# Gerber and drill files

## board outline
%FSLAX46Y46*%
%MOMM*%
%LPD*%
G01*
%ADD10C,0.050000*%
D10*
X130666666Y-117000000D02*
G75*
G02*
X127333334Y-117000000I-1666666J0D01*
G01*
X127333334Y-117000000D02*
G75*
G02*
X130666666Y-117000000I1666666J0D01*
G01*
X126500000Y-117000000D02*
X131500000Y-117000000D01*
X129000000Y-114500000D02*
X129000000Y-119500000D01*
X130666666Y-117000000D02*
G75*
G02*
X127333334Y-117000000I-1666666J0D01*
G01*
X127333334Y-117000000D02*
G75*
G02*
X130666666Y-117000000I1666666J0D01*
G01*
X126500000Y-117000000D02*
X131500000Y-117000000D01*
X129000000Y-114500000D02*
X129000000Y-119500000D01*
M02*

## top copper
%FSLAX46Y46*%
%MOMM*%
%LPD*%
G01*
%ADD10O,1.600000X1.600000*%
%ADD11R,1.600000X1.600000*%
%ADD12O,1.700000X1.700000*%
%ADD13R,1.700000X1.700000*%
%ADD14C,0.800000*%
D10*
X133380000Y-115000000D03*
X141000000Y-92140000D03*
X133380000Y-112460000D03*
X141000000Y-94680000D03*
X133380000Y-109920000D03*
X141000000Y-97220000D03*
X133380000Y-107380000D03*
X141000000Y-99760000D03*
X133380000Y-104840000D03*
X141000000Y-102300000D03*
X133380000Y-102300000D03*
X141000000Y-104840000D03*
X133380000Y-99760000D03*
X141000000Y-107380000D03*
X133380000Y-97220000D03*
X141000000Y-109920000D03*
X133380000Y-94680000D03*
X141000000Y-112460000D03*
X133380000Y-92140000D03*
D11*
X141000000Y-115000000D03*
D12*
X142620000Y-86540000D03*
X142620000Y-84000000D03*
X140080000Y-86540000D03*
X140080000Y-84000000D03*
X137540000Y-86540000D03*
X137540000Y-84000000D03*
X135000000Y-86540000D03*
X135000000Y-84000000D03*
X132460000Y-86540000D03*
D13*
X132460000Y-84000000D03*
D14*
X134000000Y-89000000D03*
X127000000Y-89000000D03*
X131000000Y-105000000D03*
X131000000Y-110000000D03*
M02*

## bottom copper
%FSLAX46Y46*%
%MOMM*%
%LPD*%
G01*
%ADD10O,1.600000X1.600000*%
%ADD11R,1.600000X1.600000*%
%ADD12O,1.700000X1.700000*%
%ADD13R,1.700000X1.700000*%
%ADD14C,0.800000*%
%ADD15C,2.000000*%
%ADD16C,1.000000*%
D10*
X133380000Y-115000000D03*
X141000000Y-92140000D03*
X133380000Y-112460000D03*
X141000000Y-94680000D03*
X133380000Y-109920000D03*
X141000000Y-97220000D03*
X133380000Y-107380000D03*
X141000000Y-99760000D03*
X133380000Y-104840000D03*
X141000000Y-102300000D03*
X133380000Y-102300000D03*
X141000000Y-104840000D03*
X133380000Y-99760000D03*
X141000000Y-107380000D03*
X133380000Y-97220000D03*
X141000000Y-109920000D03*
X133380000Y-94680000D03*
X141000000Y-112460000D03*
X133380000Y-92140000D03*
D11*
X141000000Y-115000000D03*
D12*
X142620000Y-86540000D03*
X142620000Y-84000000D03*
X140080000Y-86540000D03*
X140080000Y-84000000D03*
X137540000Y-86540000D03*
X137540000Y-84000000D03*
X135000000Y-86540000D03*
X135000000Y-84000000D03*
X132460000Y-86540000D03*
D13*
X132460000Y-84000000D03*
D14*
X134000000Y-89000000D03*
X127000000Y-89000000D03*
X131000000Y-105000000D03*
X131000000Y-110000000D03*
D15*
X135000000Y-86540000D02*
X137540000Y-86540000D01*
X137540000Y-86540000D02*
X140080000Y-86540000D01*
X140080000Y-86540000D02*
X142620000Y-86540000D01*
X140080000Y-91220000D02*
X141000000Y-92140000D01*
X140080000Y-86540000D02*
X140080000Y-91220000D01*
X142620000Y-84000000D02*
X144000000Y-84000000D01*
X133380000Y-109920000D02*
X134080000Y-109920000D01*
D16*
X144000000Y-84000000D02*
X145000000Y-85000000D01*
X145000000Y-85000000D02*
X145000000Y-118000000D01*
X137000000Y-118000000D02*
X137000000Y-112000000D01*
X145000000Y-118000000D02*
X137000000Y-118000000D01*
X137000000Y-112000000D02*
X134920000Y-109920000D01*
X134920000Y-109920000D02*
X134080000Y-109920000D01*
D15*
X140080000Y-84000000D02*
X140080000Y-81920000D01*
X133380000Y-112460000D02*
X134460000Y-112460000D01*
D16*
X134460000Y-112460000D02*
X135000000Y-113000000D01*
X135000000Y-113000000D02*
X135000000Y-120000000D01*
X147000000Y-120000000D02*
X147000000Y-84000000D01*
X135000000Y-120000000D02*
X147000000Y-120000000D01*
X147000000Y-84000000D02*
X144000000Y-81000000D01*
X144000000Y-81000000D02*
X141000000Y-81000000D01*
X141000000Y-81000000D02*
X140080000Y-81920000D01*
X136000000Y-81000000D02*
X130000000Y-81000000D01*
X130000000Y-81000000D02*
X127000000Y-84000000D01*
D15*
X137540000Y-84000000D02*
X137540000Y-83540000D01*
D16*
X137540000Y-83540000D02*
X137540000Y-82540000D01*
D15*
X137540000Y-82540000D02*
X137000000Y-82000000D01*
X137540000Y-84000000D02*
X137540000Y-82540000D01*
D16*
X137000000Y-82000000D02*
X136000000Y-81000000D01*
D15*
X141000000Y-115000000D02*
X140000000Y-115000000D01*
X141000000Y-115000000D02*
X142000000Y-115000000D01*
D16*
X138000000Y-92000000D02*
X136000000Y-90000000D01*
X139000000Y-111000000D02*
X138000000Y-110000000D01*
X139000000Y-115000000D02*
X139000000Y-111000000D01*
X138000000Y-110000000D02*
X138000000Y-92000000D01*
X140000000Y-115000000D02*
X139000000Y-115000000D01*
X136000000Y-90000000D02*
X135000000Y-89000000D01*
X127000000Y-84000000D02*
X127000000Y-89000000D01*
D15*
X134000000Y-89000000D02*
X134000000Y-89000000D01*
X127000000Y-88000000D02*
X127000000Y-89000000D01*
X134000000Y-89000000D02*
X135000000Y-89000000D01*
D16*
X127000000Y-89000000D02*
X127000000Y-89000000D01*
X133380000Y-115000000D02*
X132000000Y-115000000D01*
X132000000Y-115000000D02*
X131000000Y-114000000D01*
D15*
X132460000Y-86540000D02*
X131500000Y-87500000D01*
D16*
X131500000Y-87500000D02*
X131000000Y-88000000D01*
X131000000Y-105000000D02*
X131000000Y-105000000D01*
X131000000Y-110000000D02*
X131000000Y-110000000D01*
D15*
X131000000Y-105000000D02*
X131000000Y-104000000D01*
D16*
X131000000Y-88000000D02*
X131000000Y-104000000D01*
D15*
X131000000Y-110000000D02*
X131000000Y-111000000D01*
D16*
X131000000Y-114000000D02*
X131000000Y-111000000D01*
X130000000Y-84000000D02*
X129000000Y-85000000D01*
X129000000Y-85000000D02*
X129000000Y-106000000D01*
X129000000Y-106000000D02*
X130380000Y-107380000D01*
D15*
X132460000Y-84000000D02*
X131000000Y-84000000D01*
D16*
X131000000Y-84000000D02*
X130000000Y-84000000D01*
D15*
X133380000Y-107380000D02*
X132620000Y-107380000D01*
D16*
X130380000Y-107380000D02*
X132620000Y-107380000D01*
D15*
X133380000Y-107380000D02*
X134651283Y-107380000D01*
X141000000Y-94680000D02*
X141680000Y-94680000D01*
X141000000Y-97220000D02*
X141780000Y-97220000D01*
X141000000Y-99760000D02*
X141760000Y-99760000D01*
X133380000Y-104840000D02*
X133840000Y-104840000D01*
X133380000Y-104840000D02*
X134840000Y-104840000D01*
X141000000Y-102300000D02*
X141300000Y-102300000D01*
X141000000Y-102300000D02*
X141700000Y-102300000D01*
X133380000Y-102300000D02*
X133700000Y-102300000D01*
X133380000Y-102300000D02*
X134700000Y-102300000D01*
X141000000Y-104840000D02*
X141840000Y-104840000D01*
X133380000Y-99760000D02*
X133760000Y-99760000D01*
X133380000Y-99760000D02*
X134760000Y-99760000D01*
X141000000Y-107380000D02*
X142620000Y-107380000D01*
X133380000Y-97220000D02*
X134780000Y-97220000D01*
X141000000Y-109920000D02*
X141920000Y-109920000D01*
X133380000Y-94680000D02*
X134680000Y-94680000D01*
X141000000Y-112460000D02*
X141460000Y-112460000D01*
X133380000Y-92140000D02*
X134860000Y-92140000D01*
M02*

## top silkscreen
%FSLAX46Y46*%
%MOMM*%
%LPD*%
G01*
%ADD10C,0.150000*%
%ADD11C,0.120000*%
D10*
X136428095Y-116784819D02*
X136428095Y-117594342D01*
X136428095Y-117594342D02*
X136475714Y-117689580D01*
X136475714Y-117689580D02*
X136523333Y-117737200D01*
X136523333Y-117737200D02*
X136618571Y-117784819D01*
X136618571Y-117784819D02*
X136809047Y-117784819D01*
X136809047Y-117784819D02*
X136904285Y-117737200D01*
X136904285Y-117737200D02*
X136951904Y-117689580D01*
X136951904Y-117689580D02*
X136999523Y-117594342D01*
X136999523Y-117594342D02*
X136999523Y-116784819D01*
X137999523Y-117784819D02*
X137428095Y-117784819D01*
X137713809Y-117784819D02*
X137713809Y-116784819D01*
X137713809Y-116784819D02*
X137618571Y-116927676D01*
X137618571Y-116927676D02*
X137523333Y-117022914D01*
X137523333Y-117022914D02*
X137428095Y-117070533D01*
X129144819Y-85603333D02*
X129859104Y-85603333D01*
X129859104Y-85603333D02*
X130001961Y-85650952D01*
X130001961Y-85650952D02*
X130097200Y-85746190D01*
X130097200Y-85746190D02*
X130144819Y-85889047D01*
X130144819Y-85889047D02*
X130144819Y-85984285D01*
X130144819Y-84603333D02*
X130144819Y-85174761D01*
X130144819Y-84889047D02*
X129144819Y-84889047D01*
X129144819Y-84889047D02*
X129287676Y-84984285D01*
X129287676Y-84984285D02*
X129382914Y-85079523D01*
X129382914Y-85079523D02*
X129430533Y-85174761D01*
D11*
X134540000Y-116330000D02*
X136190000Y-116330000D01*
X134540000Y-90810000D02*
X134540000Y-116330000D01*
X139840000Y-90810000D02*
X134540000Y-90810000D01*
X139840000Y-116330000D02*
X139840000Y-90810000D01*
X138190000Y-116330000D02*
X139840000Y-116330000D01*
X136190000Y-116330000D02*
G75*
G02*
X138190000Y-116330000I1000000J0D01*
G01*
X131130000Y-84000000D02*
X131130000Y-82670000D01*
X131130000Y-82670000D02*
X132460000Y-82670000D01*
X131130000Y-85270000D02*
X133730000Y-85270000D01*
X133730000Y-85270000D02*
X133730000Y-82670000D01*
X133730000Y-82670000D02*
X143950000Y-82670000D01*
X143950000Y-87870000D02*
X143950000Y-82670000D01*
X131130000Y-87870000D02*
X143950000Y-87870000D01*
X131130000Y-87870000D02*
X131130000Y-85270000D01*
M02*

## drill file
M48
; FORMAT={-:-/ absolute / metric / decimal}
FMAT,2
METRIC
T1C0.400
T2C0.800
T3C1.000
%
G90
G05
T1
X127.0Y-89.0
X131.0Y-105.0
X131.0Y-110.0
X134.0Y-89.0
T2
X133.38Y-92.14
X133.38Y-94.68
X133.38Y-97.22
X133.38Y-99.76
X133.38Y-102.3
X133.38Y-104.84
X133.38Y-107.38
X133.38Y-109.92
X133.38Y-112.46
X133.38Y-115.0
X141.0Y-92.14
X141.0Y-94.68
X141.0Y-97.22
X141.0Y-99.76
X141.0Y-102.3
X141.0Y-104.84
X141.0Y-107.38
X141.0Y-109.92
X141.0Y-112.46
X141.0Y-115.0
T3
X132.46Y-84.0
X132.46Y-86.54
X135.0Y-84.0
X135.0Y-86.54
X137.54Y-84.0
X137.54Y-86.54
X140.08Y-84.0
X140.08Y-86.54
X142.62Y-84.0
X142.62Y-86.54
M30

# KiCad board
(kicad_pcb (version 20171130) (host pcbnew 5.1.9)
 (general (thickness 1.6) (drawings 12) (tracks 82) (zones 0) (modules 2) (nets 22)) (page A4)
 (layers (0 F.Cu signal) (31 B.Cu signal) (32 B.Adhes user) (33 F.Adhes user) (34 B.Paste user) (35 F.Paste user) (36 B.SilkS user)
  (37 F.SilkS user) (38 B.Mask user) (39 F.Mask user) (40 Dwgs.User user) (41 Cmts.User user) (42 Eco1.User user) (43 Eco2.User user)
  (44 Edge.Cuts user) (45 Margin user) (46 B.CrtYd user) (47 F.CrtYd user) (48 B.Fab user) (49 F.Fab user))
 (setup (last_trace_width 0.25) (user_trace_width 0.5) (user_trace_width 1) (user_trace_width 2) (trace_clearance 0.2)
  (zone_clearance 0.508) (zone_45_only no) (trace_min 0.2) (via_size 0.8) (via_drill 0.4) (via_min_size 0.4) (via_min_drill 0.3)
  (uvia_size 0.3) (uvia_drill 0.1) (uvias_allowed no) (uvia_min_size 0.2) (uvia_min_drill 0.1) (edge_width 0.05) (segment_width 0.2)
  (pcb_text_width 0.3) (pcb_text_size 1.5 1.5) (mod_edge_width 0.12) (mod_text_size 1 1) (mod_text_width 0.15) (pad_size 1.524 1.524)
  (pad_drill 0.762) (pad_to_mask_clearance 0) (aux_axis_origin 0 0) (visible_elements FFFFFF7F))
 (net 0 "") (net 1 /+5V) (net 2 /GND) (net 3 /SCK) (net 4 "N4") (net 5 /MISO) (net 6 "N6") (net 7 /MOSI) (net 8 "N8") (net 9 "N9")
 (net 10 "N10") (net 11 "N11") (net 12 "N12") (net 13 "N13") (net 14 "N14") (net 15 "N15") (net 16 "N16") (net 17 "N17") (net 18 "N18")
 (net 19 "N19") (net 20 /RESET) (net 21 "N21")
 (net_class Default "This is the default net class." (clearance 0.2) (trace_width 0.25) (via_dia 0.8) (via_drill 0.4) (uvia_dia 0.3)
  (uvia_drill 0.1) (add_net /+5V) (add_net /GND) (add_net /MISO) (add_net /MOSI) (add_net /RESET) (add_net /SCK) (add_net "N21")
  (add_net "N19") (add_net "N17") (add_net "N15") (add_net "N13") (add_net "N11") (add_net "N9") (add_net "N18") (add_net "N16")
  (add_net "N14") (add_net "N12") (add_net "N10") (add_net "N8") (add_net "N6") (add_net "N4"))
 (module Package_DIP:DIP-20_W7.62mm (layer F.Cu) (at 141 115 180)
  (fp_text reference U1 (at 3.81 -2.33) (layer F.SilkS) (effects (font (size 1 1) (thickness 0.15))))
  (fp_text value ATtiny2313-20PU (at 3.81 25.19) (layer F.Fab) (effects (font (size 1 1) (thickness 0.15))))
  (fp_line (start 6.46 -1.33) (end 4.81 -1.33) (layer F.SilkS) (width 0.12))
  (fp_line (start 6.46 24.19) (end 6.46 -1.33) (layer F.SilkS) (width 0.12))
  (fp_line (start 1.16 24.19) (end 6.46 24.19) (layer F.SilkS) (width 0.12))
  (fp_line (start 1.16 -1.33) (end 1.16 24.19) (layer F.SilkS) (width 0.12))
  (fp_line (start 2.81 -1.33) (end 1.16 -1.33) (layer F.SilkS) (width 0.12))
  (fp_arc (start 3.81 -1.33) (end 2.81 -1.33) (angle -180) (layer F.SilkS) (width 0.12))
  (pad 20 thru_hole oval (at 7.62 0 180) (size 1.6 1.6) (drill 0.8) (layers *.Cu *.Mask) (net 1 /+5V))
  (pad 10 thru_hole oval (at 0 22.86 180) (size 1.6 1.6) (drill 0.8) (layers *.Cu *.Mask) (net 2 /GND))
  (pad 19 thru_hole oval (at 7.62 2.54 180) (size 1.6 1.6) (drill 0.8) (layers *.Cu *.Mask) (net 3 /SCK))
  (pad 9 thru_hole oval (at 0 20.32 180) (size 1.6 1.6) (drill 0.8) (layers *.Cu *.Mask) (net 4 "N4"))
  (pad 18 thru_hole oval (at 7.62 5.08 180) (size 1.6 1.6) (drill 0.8) (layers *.Cu *.Mask) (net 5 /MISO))
  (pad 8 thru_hole oval (at 0 17.78 180) (size 1.6 1.6) (drill 0.8) (layers *.Cu *.Mask) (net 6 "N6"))
  (pad 17 thru_hole oval (at 7.62 7.62 180) (size 1.6 1.6) (drill 0.8) (layers *.Cu *.Mask) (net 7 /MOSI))
  (pad 7 thru_hole oval (at 0 15.24 180) (size 1.6 1.6) (drill 0.8) (layers *.Cu *.Mask) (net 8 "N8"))
  (pad 16 thru_hole oval (at 7.62 10.16 180) (size 1.6 1.6) (drill 0.8) (layers *.Cu *.Mask) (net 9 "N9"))
  (pad 6 thru_hole oval (at 0 12.7 180) (size 1.6 1.6) (drill 0.8) (layers *.Cu *.Mask) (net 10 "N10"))
  (pad 15 thru_hole oval (at 7.62 12.7 180) (size 1.6 1.6) (drill 0.8) (layers *.Cu *.Mask) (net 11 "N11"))
  (pad 5 thru_hole oval (at 0 10.16 180) (size 1.6 1.6) (drill 0.8) (layers *.Cu *.Mask) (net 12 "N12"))
  (pad 14 thru_hole oval (at 7.62 15.24 180) (size 1.6 1.6) (drill 0.8) (layers *.Cu *.Mask) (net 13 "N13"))
  (pad 4 thru_hole oval (at 0 7.62 180) (size 1.6 1.6) (drill 0.8) (layers *.Cu *.Mask) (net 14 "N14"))
  (pad 13 thru_hole oval (at 7.62 17.78 180) (size 1.6 1.6) (drill 0.8) (layers *.Cu *.Mask) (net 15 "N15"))
  (pad 3 thru_hole oval (at 0 5.08 180) (size 1.6 1.6) (drill 0.8) (layers *.Cu *.Mask) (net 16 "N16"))
  (pad 12 thru_hole oval (at 7.62 20.32 180) (size 1.6 1.6) (drill 0.8) (layers *.Cu *.Mask) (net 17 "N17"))
  (pad 2 thru_hole oval (at 0 2.54 180) (size 1.6 1.6) (drill 0.8) (layers *.Cu *.Mask) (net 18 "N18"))
  (pad 11 thru_hole oval (at 7.62 22.86 180) (size 1.6 1.6) (drill 0.8) (layers *.Cu *.Mask) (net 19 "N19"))
  (pad 1 thru_hole rect (at 0 0 180) (size 1.6 1.6) (drill 0.8) (layers *.Cu *.Mask) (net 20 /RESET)))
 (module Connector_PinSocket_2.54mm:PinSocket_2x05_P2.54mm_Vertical (layer F.Cu) (at 132.46 84 90)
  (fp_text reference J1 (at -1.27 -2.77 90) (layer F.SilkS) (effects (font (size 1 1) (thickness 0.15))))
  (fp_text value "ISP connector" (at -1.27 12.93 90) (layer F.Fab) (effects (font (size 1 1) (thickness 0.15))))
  (fp_line (start 0 -1.33) (end 1.33 -1.33) (layer F.SilkS) (width 0.12))
  (fp_line (start 1.33 -1.33) (end 1.33 0) (layer F.SilkS) (width 0.12))
  (fp_line (start -1.27 -1.33) (end -1.27 1.27) (layer F.SilkS) (width 0.12))
  (fp_line (start -1.27 1.27) (end 1.33 1.27) (layer F.SilkS) (width 0.12))
  (fp_line (start 1.33 1.27) (end 1.33 11.49) (layer F.SilkS) (width 0.12))
  (fp_line (start -3.87 11.49) (end 1.33 11.49) (layer F.SilkS) (width 0.12))
  (fp_line (start -3.87 -1.33) (end -3.87 11.49) (layer F.SilkS) (width 0.12))
  (fp_line (start -3.87 -1.33) (end -1.27 -1.33) (layer F.SilkS) (width 0.12))
  (pad 10 thru_hole oval (at -2.54 10.16 90) (size 1.7 1.7) (drill 1) (layers *.Cu *.Mask) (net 2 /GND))
  (pad 9 thru_hole oval (at 0 10.16 90) (size 1.7 1.7) (drill 1) (layers *.Cu *.Mask) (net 5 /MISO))
  (pad 8 thru_hole oval (at -2.54 7.62 90) (size 1.7 1.7) (drill 1) (layers *.Cu *.Mask) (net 2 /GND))
  (pad 7 thru_hole oval (at 0 7.62 90) (size 1.7 1.7) (drill 1) (layers *.Cu *.Mask) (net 3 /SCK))
  (pad 6 thru_hole oval (at -2.54 5.08 90) (size 1.7 1.7) (drill 1) (layers *.Cu *.Mask) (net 2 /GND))
  (pad 5 thru_hole oval (at 0 5.08 90) (size 1.7 1.7) (drill 1) (layers *.Cu *.Mask) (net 20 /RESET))
  (pad 4 thru_hole oval (at -2.54 2.54 90) (size 1.7 1.7) (drill 1) (layers *.Cu *.Mask) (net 2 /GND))
  (pad 3 thru_hole oval (at 0 2.54 90) (size 1.7 1.7) (drill 1) (layers *.Cu *.Mask) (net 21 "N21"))
  (pad 2 thru_hole oval (at -2.54 0 90) (size 1.7 1.7) (drill 1) (layers *.Cu *.Mask) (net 1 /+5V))
  (pad 1 thru_hole rect (at 0 0 90) (size 1.7 1.7) (drill 1) (layers *.Cu *.Mask) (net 7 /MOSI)))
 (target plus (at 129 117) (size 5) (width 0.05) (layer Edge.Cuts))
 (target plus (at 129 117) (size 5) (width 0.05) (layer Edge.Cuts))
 (segment (start 135 86.54) (end 137.54 86.54) (width 2) (layer B.Cu) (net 2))
 (segment (start 137.54 86.54) (end 140.08 86.54) (width 2) (layer B.Cu) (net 2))
 (segment (start 140.08 86.54) (end 142.62 86.54) (width 2) (layer B.Cu) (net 2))
 (segment (start 140.08 91.22) (end 141 92.14) (width 2) (layer B.Cu) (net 2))
 (segment (start 140.08 86.54) (end 140.08 91.22) (width 2) (layer B.Cu) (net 2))
 (segment (start 142.62 84) (end 144 84) (width 2) (layer B.Cu) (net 5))
 (segment (start 133.38 109.92) (end 134.08 109.92) (width 2) (layer B.Cu) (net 5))
 (segment (start 144 84) (end 145 85) (width 1) (layer B.Cu) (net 5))
 (segment (start 145 85) (end 145 118) (width 1) (layer B.Cu) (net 5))
 (segment (start 137 118) (end 137 112) (width 1) (layer B.Cu) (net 5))
 (segment (start 145 118) (end 137 118) (width 1) (layer B.Cu) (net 5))
 (segment (start 137 112) (end 134.92 109.92) (width 1) (layer B.Cu) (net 5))
 (segment (start 134.92 109.92) (end 134.08 109.92) (width 1) (layer B.Cu) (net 5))
 (segment (start 140.08 84) (end 140.08 81.92) (width 2) (layer B.Cu) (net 3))
 (segment (start 133.38 112.46) (end 134.46 112.46) (width 2) (layer B.Cu) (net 3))
 (segment (start 134.46 112.46) (end 135 113) (width 1) (layer B.Cu) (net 3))
 (segment (start 135 113) (end 135 120) (width 1) (layer B.Cu) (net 3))
 (segment (start 147 120) (end 147 84) (width 1) (layer B.Cu) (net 3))
 (segment (start 135 120) (end 147 120) (width 1) (layer B.Cu) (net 3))
 (segment (start 147 84) (end 144 81) (width 1) (layer B.Cu) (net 3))
 (segment (start 144 81) (end 141 81) (width 1) (layer B.Cu) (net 3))
 (segment (start 141 81) (end 140.08 81.92) (width 1) (layer B.Cu) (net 3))
 (segment (start 136 81) (end 130 81) (width 1) (layer B.Cu) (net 20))
 (segment (start 130 81) (end 127 84) (width 1) (layer B.Cu) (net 20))
 (segment (start 137.54 84) (end 137.54 83.54) (width 2) (layer B.Cu) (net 20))
 (segment (start 137.54 83.54) (end 137.54 82.54) (width 1) (layer B.Cu) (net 20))
 (segment (start 137.54 82.54) (end 137 82) (width 2) (layer B.Cu) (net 20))
 (segment (start 137.54 84) (end 137.54 82.54) (width 2) (layer B.Cu) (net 20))
 (segment (start 137 82) (end 136 81) (width 1) (layer B.Cu) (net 20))
 (segment (start 141 115) (end 140 115) (width 2) (layer B.Cu) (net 20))
 (segment (start 141 115) (end 142 115) (width 2) (layer B.Cu) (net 20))
 (segment (start 138 92) (end 136 90) (width 1) (layer B.Cu) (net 20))
 (segment (start 139 111) (end 138 110) (width 1) (layer B.Cu) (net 20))
 (segment (start 139 115) (end 139 111) (width 1) (layer B.Cu) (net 20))
 (segment (start 138 110) (end 138 92) (width 1) (layer B.Cu) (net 20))
 (segment (start 140 115) (end 139 115) (width 1) (layer B.Cu) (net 20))
 (segment (start 136 90) (end 135 89) (width 1) (layer B.Cu) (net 20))
 (segment (start 127 84) (end 127 89) (width 1) (layer B.Cu) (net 20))
 (segment (start 134 89) (end 134 89) (width 2) (layer B.Cu) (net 20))
 (segment (start 127 88) (end 127 89) (width 2) (layer B.Cu) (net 20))
 (segment (start 134 89) (end 135 89) (width 2) (layer B.Cu) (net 20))
 (via (at 134 89) (size 0.8) (drill 0.4) (layers F.Cu B.Cu) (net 20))
 (segment (start 127 89) (end 127 89) (width 1) (layer B.Cu) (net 20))
 (via (at 127 89) (size 0.8) (drill 0.4) (layers F.Cu B.Cu) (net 20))
 (segment (start 133.38 115) (end 132 115) (width 1) (layer B.Cu) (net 1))
 (segment (start 132 115) (end 131 114) (width 1) (layer B.Cu) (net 1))
 (segment (start 132.46 86.54) (end 131.5 87.5) (width 2) (layer B.Cu) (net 1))
 (segment (start 131.5 87.5) (end 131 88) (width 1) (layer B.Cu) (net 1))
 (segment (start 131 105) (end 131 105) (width 1) (layer B.Cu) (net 1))
 (via (at 131 105) (size 0.8) (drill 0.4) (layers F.Cu B.Cu) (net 1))
 (segment (start 131 110) (end 131 110) (width 1) (layer B.Cu) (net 1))
 (via (at 131 110) (size 0.8) (drill 0.4) (layers F.Cu B.Cu) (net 1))
 (segment (start 131 105) (end 131 104) (width 2) (layer B.Cu) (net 1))
 (segment (start 131 88) (end 131 104) (width 1) (layer B.Cu) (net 1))
 (segment (start 131 110) (end 131 111) (width 2) (layer B.Cu) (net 1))
 (segment (start 131 114) (end 131 111) (width 1) (layer B.Cu) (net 1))
 (segment (start 130 84) (end 129 85) (width 1) (layer B.Cu) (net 7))
 (segment (start 129 85) (end 129 106) (width 1) (layer B.Cu) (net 7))
 (segment (start 129 106) (end 130.38 107.38) (width 1) (layer B.Cu) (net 7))
 (segment (start 132.46 84) (end 131 84) (width 2) (layer B.Cu) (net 7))
 (segment (start 131 84) (end 130 84) (width 1) (layer B.Cu) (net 7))
 (segment (start 133.38 107.38) (end 132.62 107.38) (width 2) (layer B.Cu) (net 7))
 (segment (start 130.38 107.38) (end 132.62 107.38) (width 1) (layer B.Cu) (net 7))
 (segment (start 133.38 107.38) (end 134.651283 107.38) (width 2) (layer B.Cu) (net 7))
 (segment (start 141 94.68) (end 141.68 94.68) (width 2) (layer B.Cu) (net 4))
 (segment (start 141 97.22) (end 141.78 97.22) (width 2) (layer B.Cu) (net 6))
 (segment (start 141 99.76) (end 141.76 99.76) (width 2) (layer B.Cu) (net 8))
 (segment (start 133.38 104.84) (end 133.84 104.84) (width 2) (layer B.Cu) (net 9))
 (segment (start 133.38 104.84) (end 134.84 104.84) (width 2) (layer B.Cu) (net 9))
 (segment (start 141 102.3) (end 141.3 102.3) (width 2) (layer B.Cu) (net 10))
 (segment (start 141 102.3) (end 141.7 102.3) (width 2) (layer B.Cu) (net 10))
 (segment (start 133.38 102.3) (end 133.7 102.3) (width 2) (layer B.Cu) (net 11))
 (segment (start 133.38 102.3) (end 134.7 102.3) (width 2) (layer B.Cu) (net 11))
 (segment (start 141 104.84) (end 141.84 104.84) (width 2) (layer B.Cu) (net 12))
 (segment (start 133.38 99.76) (end 133.76 99.76) (width 2) (layer B.Cu) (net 13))
 (segment (start 133.38 99.76) (end 134.76 99.76) (width 2) (layer B.Cu) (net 13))
 (segment (start 141 107.38) (end 142.62 107.38) (width 2) (layer B.Cu) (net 14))
 (segment (start 133.38 97.22) (end 134.78 97.22) (width 2) (layer B.Cu) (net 15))
 (segment (start 141 109.92) (end 141.92 109.92) (width 2) (layer B.Cu) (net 16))
 (segment (start 133.38 94.68) (end 134.68 94.68) (width 2) (layer B.Cu) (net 17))
 (segment (start 141 112.46) (end 141.46 112.46) (width 2) (layer B.Cu) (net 18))
 (segment (start 133.38 92.14) (end 134.86 92.14) (width 2) (layer B.Cu) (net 19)))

